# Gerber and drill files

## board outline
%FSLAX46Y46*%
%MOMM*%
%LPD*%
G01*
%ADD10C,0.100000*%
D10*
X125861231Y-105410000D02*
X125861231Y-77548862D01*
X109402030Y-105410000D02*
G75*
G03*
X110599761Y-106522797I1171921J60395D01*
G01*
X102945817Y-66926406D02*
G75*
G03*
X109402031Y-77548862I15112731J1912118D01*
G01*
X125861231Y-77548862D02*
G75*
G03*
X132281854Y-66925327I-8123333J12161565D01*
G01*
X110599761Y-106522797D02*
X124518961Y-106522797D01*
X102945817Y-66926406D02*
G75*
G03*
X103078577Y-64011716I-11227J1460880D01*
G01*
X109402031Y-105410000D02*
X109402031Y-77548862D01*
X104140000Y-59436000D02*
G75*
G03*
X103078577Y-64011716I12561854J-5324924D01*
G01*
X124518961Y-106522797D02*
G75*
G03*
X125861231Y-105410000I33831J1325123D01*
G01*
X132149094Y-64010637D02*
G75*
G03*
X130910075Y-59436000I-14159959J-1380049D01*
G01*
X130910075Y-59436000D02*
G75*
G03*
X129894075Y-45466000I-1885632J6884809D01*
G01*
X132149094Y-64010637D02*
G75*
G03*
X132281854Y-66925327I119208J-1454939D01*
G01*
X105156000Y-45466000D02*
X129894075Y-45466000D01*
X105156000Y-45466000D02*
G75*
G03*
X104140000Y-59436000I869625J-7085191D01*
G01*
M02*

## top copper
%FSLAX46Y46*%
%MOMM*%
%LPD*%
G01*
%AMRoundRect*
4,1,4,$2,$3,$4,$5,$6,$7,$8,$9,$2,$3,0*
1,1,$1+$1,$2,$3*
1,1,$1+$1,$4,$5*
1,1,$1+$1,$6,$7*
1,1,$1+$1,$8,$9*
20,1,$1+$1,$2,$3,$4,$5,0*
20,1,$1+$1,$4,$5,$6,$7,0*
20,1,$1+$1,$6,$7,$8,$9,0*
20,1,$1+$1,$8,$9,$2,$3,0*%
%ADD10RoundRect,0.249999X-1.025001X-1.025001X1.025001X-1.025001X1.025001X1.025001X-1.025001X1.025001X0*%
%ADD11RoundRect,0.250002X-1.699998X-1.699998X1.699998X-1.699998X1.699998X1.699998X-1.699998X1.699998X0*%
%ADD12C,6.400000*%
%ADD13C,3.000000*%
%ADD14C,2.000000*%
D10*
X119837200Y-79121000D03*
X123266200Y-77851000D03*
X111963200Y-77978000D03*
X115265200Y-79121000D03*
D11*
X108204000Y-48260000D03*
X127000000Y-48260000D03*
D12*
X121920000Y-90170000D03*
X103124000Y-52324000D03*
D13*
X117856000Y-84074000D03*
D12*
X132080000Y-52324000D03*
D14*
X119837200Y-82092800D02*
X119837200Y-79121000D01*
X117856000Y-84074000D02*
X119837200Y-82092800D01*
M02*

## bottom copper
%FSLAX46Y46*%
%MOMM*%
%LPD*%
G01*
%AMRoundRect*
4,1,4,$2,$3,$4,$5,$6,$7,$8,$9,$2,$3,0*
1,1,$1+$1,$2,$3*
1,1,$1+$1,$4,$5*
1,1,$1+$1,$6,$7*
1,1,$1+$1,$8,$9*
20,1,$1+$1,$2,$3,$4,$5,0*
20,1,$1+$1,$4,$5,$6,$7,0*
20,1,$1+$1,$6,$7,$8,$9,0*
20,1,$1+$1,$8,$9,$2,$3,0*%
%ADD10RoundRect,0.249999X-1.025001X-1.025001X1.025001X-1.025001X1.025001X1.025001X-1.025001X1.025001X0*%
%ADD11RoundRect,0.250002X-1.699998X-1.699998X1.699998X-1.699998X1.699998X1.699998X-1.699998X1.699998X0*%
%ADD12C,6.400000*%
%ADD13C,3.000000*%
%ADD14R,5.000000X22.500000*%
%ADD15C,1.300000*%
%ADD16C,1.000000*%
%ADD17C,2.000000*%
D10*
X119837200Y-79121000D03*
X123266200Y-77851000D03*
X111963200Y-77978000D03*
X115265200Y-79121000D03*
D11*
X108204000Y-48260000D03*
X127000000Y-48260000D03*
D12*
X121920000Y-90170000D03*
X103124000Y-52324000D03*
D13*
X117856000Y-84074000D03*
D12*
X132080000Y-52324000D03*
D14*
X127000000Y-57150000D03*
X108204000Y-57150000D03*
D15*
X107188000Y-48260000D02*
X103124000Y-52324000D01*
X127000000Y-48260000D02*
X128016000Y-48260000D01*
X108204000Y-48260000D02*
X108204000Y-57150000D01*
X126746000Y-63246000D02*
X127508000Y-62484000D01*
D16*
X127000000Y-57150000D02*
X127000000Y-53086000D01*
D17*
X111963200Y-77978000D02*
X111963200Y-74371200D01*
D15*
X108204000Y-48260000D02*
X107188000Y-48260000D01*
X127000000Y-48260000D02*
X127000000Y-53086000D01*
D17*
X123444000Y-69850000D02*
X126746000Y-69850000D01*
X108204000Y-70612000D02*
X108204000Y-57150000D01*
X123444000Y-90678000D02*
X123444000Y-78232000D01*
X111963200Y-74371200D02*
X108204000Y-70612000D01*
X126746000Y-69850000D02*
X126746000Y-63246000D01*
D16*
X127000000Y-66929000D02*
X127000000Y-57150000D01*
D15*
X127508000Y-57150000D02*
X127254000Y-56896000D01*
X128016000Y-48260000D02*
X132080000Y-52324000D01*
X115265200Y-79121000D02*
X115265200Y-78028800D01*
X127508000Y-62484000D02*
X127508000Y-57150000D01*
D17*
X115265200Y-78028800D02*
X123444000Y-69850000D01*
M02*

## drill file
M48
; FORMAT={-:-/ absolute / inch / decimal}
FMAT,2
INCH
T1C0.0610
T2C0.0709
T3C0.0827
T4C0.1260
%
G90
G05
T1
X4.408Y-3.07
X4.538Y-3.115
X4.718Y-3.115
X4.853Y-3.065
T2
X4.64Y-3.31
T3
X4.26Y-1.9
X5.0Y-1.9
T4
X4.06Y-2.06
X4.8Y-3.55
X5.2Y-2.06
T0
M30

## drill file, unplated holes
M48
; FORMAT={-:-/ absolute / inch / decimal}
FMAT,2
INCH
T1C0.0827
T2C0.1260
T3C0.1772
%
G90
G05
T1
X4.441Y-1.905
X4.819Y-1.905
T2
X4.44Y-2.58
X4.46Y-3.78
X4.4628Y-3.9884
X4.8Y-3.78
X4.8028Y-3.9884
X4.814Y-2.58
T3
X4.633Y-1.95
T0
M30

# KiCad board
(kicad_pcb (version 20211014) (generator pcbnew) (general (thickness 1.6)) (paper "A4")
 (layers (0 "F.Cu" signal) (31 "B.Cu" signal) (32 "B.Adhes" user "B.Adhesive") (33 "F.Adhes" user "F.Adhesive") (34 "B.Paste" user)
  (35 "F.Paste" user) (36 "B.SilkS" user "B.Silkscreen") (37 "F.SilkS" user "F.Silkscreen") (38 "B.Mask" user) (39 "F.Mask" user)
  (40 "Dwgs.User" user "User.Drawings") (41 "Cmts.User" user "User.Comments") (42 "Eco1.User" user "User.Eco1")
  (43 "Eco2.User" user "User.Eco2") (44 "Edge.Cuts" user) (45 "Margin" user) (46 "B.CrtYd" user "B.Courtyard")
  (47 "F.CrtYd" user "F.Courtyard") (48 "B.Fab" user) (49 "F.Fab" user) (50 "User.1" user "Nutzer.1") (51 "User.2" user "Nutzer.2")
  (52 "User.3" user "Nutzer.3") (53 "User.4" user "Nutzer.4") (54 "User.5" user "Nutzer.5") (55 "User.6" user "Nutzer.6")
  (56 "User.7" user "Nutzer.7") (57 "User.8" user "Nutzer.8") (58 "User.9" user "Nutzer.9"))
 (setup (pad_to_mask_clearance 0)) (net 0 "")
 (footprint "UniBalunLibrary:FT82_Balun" (layer "F.Cu") (at 117.602 65.532)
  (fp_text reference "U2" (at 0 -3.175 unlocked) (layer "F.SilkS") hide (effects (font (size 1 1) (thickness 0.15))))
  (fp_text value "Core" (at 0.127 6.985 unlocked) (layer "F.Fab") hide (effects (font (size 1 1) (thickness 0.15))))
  (pad "" np_thru_hole circle (at -4.826 0) (size 3.2 3.2) (drill 3.2) (layers *.Cu *.Mask))
  (pad "" np_thru_hole circle (at 4.6736 0) (size 3.2 3.2) (drill 3.2) (layers *.Cu *.Mask))
  (pad "1" thru_hole roundrect (at 2.2352 13.589) (size 2.55 2.55) (drill 1.55) (layers *.Cu *.Mask) (roundrect_rratio 0.09803882353))
  (pad "2" thru_hole roundrect (at 5.6642 12.319) (size 2.55 2.55) (drill 1.55) (layers *.Cu *.Mask) (roundrect_rratio 0.09803882353))
  (pad "3" thru_hole roundrect (at -5.6388 12.446) (size 2.55 2.55) (drill 1.55) (layers *.Cu *.Mask) (roundrect_rratio 0.09803882353))
  (pad "4" thru_hole roundrect (at -2.3368 13.589) (size 2.55 2.55) (drill 1.55) (layers *.Cu *.Mask) (roundrect_rratio 0.09803882353)))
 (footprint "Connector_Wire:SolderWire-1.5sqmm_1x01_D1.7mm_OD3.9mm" (layer "F.Cu") (at 108.204 48.26)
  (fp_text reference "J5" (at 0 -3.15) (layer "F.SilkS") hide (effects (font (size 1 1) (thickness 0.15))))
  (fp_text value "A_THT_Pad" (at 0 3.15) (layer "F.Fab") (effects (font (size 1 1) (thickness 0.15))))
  (pad "1" thru_hole roundrect (at 0 0) (size 3.9 3.9) (drill 2.1) (layers *.Cu *.Mask) (roundrect_rratio 0.06410307692)))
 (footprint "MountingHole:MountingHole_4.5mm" (layer "F.Cu") (at 117.6782 49.53)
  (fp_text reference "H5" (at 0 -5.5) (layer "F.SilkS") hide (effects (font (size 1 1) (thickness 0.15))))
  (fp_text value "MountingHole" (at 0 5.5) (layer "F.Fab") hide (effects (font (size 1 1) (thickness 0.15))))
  (pad "" np_thru_hole circle (at 0 0) (size 4.5 4.5) (drill 4.5) (layers *.Cu *.Mask)))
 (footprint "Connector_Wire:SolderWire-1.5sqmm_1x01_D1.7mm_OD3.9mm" (layer "F.Cu") (at 127 48.26)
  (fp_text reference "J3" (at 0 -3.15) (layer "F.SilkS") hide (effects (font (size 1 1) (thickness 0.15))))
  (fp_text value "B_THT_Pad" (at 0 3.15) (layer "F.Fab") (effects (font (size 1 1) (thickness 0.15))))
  (pad "1" thru_hole roundrect (at 0 0) (size 3.9 3.9) (drill 2.1) (layers *.Cu *.Mask) (roundrect_rratio 0.06410307692)))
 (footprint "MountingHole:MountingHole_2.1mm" (layer "F.Cu") (at 112.8014 48.387)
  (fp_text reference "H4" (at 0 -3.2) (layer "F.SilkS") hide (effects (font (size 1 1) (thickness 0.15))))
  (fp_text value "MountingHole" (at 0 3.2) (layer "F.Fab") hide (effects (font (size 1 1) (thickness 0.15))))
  (pad "" np_thru_hole circle (at 0 0) (size 2.1 2.1) (drill 2.1) (layers *.Cu *.Mask)))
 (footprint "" (layer "F.Cu") (at 121.92 90.17)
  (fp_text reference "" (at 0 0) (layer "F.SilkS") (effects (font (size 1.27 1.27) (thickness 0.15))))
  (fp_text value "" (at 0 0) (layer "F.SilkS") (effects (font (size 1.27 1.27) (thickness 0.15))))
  (pad "1" thru_hole circle (at 0 0) (size 6.4 6.4) (drill 3.2) (layers *.Cu *.Mask)))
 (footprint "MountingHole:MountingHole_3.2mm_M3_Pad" (layer "F.Cu") (at 103.124 52.324)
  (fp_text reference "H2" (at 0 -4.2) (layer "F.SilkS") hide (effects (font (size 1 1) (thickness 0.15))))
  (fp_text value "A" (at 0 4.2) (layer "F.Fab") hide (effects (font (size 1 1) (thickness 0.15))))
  (pad "1" thru_hole circle (at 0 0) (size 6.4 6.4) (drill 3.2) (layers *.Cu *.Mask)))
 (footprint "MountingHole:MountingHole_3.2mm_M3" (layer "F.Cu") (at 121.991969 101.306569)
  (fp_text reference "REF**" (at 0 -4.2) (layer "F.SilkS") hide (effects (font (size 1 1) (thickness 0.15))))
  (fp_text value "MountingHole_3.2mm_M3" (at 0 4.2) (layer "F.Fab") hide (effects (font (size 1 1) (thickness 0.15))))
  (pad "" np_thru_hole circle (at 0 0) (size 3.2 3.2) (drill 3.2) (layers *.Cu *.Mask)))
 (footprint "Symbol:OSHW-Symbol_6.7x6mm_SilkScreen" (layer "F.Cu") (at 117.6 68.6)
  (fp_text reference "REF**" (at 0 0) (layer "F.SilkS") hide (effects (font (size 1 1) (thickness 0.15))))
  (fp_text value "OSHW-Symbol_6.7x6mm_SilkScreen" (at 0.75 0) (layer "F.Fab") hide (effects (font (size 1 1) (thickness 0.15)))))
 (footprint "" (layer "F.Cu") (at 117.856 84.074)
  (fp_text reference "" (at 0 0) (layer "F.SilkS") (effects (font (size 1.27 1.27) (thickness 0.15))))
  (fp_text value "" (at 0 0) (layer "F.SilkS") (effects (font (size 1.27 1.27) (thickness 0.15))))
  (pad "1" thru_hole circle (at 0 0) (size 3 3) (drill 1.8) (layers *.Cu *.Mask)))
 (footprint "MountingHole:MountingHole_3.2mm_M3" (layer "F.Cu") (at 113.284 96.012)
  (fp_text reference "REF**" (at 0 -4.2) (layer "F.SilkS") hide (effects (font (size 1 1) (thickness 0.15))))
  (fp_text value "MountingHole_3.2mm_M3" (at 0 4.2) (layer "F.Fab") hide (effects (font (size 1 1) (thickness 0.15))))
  (pad "" np_thru_hole circle (at 0 0) (size 3.2 3.2) (drill 3.2) (layers *.Cu *.Mask)))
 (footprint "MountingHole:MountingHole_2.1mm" (layer "F.Cu") (at 122.4026 48.387)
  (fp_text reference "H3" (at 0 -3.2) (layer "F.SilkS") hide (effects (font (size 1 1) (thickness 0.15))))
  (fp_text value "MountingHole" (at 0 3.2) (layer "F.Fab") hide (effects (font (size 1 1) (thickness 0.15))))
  (pad "" np_thru_hole circle (at 0 0) (size 2.1 2.1) (drill 2.1) (layers *.Cu *.Mask)))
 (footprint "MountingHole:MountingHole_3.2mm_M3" (layer "F.Cu") (at 113.355969 101.306569)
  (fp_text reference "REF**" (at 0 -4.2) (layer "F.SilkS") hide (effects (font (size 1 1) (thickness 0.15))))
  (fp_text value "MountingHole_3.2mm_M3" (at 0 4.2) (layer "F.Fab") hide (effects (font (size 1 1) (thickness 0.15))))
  (pad "" np_thru_hole circle (at 0 0) (size 3.2 3.2) (drill 3.2) (layers *.Cu *.Mask)))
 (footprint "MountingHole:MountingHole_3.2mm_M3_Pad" (layer "F.Cu") (at 132.08 52.324)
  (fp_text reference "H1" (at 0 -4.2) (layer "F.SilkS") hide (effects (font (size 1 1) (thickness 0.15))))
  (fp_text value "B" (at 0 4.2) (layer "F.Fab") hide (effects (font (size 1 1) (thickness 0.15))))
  (pad "1" thru_hole circle (at 0 0) (size 6.4 6.4) (drill 3.2) (layers *.Cu *.Mask)))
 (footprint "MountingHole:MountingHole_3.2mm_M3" (layer "F.Cu") (at 121.92 96.012)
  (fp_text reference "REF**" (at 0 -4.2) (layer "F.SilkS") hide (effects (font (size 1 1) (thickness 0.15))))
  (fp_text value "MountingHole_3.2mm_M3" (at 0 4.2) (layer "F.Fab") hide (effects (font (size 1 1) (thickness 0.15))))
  (pad "" np_thru_hole circle (at 0 0) (size 3.2 3.2) (drill 3.2) (layers *.Cu *.Mask)))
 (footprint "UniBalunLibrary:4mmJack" (layer "B.Cu") (at 127.254 56.896 90)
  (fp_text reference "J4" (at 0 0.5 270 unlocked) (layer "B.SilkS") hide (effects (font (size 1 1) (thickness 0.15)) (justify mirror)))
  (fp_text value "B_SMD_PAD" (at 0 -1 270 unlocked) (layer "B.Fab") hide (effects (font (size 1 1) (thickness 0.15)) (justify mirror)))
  (pad "1" smd rect (at -0.254 -0.254 90) (size 22.5 5) (layers "B.Cu" "B.Mask")))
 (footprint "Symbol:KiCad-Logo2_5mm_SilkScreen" (layer "B.Cu") (at 117.729 58.547 180)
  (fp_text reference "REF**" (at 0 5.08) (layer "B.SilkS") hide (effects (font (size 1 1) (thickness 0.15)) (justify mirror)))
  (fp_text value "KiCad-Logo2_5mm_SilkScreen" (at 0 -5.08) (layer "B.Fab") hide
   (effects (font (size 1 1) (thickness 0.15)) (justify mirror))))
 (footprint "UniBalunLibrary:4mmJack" (layer "B.Cu") (at 108.458 56.896 90)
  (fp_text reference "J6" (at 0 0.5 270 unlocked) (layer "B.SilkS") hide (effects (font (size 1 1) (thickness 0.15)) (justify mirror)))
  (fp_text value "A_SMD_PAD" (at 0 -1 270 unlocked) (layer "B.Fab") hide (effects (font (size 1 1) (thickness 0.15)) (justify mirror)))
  (pad "1" smd rect (at -0.254 -0.254 90) (size 22.5 5) (layers "B.Cu" "B.Mask")))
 (gr_line (start 125.861231 105.41) (end 125.861231 77.548862) (layer "Edge.Cuts") (width 0.1))
 (gr_arc (start 110.599761 106.522797) (mid 109.77522 106.209299) (end 109.402031 105.41) (layer "Edge.Cuts") (width 0.1))
 (gr_arc (start 109.402031 77.548862) (mid 105.04112 72.92614) (end 102.945817 66.926406) (layer "Edge.Cuts") (width 0.1))
 (gr_arc (start 132.281854 66.925327) (mid 130.254542 72.952072) (end 125.861231 77.548862) (layer "Edge.Cuts") (width 0.1))
 (gr_line (start 110.599761 106.522797) (end 124.518961 106.522797) (layer "Edge.Cuts") (width 0.1))
 (gr_arc (start 103.078577 64.011716) (mid 104.394 65.532) (end 102.945817 66.926406) (layer "Edge.Cuts") (width 0.1))
 (gr_line (start 109.402031 105.41) (end 109.402031 77.548862) (layer "Edge.Cuts") (width 0.1))
 (gr_arc (start 103.078577 64.011716) (mid 103.410896 61.677837) (end 104.14 59.436) (layer "Edge.Cuts") (width 0.1))
 (gr_arc (start 125.861231 105.41) (mid 125.398804 106.218144) (end 124.518961 106.522797) (layer "Edge.Cuts") (width 0.1))
 (gr_arc (start 130.910075 59.436) (mid 131.721418 61.671361) (end 132.149094 64.010637) (layer "Edge.Cuts") (width 0.1))
 (gr_arc (start 129.894075 45.466) (mid 136.144 52.033405) (end 130.910075 59.436) (layer "Edge.Cuts") (width 0.1))
 (gr_arc (start 132.281854 66.925327) (mid 130.81 65.532) (end 132.149094 64.010637) (layer "Edge.Cuts") (width 0.1))
 (gr_line (start 105.156 45.466) (end 129.894075 45.466) (layer "Edge.Cuts") (width 0.1))
 (gr_arc (start 104.14 59.436) (mid 98.906069 52.033405) (end 105.156 45.466) (layer "Edge.Cuts") (width 0.1))
 (segment (start 119.8372 82.0928) (end 119.8372 79.121) (width 2) (layer "F.Cu") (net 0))
 (segment (start 117.856 84.074) (end 119.8372 82.0928) (width 2) (layer "F.Cu") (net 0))
 (segment (start 107.188 48.26) (end 103.124 52.324) (width 1.3) (layer "B.Cu") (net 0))
 (segment (start 127 48.26) (end 128.016 48.26) (width 1.3) (layer "B.Cu") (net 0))
 (segment (start 108.204 48.26) (end 108.204 57.15) (width 1.3) (layer "B.Cu") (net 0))
 (segment (start 126.746 63.246) (end 127.508 62.484) (width 1.3) (layer "B.Cu") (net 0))
 (segment (start 127 57.15) (end 127 53.086) (width 1) (layer "B.Cu") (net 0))
 (segment (start 111.9632 77.978) (end 111.9632 74.3712) (width 2) (layer "B.Cu") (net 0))
 (segment (start 108.204 48.26) (end 107.188 48.26) (width 1.3) (layer "B.Cu") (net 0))
 (segment (start 127 48.26) (end 127 53.086) (width 1.3) (layer "B.Cu") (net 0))
 (segment (start 123.444 69.85) (end 126.746 69.85) (width 2) (layer "B.Cu") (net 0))
 (segment (start 108.204 70.612) (end 108.204 57.15) (width 2) (layer "B.Cu") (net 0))
 (segment (start 123.444 90.678) (end 123.444 78.232) (width 2) (layer "B.Cu") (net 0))
 (segment (start 111.9632 74.3712) (end 108.204 70.612) (width 2) (layer "B.Cu") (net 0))
 (segment (start 126.746 69.85) (end 126.746 63.246) (width 2) (layer "B.Cu") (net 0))
 (segment (start 127 66.929) (end 127 57.15) (width 1) (layer "B.Cu") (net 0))
 (segment (start 127.508 57.15) (end 127.254 56.896) (width 1.3) (layer "B.Cu") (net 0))
 (segment (start 128.016 48.26) (end 132.08 52.324) (width 1.3) (layer "B.Cu") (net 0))
 (segment (start 115.2652 79.121) (end 115.2652 78.0288) (width 1.3) (layer "B.Cu") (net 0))
 (segment (start 127.508 62.484) (end 127.508 57.15) (width 1.3) (layer "B.Cu") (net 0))
 (segment (start 115.2652 78.0288) (end 123.444 69.85) (width 2) (layer "B.Cu") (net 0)))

